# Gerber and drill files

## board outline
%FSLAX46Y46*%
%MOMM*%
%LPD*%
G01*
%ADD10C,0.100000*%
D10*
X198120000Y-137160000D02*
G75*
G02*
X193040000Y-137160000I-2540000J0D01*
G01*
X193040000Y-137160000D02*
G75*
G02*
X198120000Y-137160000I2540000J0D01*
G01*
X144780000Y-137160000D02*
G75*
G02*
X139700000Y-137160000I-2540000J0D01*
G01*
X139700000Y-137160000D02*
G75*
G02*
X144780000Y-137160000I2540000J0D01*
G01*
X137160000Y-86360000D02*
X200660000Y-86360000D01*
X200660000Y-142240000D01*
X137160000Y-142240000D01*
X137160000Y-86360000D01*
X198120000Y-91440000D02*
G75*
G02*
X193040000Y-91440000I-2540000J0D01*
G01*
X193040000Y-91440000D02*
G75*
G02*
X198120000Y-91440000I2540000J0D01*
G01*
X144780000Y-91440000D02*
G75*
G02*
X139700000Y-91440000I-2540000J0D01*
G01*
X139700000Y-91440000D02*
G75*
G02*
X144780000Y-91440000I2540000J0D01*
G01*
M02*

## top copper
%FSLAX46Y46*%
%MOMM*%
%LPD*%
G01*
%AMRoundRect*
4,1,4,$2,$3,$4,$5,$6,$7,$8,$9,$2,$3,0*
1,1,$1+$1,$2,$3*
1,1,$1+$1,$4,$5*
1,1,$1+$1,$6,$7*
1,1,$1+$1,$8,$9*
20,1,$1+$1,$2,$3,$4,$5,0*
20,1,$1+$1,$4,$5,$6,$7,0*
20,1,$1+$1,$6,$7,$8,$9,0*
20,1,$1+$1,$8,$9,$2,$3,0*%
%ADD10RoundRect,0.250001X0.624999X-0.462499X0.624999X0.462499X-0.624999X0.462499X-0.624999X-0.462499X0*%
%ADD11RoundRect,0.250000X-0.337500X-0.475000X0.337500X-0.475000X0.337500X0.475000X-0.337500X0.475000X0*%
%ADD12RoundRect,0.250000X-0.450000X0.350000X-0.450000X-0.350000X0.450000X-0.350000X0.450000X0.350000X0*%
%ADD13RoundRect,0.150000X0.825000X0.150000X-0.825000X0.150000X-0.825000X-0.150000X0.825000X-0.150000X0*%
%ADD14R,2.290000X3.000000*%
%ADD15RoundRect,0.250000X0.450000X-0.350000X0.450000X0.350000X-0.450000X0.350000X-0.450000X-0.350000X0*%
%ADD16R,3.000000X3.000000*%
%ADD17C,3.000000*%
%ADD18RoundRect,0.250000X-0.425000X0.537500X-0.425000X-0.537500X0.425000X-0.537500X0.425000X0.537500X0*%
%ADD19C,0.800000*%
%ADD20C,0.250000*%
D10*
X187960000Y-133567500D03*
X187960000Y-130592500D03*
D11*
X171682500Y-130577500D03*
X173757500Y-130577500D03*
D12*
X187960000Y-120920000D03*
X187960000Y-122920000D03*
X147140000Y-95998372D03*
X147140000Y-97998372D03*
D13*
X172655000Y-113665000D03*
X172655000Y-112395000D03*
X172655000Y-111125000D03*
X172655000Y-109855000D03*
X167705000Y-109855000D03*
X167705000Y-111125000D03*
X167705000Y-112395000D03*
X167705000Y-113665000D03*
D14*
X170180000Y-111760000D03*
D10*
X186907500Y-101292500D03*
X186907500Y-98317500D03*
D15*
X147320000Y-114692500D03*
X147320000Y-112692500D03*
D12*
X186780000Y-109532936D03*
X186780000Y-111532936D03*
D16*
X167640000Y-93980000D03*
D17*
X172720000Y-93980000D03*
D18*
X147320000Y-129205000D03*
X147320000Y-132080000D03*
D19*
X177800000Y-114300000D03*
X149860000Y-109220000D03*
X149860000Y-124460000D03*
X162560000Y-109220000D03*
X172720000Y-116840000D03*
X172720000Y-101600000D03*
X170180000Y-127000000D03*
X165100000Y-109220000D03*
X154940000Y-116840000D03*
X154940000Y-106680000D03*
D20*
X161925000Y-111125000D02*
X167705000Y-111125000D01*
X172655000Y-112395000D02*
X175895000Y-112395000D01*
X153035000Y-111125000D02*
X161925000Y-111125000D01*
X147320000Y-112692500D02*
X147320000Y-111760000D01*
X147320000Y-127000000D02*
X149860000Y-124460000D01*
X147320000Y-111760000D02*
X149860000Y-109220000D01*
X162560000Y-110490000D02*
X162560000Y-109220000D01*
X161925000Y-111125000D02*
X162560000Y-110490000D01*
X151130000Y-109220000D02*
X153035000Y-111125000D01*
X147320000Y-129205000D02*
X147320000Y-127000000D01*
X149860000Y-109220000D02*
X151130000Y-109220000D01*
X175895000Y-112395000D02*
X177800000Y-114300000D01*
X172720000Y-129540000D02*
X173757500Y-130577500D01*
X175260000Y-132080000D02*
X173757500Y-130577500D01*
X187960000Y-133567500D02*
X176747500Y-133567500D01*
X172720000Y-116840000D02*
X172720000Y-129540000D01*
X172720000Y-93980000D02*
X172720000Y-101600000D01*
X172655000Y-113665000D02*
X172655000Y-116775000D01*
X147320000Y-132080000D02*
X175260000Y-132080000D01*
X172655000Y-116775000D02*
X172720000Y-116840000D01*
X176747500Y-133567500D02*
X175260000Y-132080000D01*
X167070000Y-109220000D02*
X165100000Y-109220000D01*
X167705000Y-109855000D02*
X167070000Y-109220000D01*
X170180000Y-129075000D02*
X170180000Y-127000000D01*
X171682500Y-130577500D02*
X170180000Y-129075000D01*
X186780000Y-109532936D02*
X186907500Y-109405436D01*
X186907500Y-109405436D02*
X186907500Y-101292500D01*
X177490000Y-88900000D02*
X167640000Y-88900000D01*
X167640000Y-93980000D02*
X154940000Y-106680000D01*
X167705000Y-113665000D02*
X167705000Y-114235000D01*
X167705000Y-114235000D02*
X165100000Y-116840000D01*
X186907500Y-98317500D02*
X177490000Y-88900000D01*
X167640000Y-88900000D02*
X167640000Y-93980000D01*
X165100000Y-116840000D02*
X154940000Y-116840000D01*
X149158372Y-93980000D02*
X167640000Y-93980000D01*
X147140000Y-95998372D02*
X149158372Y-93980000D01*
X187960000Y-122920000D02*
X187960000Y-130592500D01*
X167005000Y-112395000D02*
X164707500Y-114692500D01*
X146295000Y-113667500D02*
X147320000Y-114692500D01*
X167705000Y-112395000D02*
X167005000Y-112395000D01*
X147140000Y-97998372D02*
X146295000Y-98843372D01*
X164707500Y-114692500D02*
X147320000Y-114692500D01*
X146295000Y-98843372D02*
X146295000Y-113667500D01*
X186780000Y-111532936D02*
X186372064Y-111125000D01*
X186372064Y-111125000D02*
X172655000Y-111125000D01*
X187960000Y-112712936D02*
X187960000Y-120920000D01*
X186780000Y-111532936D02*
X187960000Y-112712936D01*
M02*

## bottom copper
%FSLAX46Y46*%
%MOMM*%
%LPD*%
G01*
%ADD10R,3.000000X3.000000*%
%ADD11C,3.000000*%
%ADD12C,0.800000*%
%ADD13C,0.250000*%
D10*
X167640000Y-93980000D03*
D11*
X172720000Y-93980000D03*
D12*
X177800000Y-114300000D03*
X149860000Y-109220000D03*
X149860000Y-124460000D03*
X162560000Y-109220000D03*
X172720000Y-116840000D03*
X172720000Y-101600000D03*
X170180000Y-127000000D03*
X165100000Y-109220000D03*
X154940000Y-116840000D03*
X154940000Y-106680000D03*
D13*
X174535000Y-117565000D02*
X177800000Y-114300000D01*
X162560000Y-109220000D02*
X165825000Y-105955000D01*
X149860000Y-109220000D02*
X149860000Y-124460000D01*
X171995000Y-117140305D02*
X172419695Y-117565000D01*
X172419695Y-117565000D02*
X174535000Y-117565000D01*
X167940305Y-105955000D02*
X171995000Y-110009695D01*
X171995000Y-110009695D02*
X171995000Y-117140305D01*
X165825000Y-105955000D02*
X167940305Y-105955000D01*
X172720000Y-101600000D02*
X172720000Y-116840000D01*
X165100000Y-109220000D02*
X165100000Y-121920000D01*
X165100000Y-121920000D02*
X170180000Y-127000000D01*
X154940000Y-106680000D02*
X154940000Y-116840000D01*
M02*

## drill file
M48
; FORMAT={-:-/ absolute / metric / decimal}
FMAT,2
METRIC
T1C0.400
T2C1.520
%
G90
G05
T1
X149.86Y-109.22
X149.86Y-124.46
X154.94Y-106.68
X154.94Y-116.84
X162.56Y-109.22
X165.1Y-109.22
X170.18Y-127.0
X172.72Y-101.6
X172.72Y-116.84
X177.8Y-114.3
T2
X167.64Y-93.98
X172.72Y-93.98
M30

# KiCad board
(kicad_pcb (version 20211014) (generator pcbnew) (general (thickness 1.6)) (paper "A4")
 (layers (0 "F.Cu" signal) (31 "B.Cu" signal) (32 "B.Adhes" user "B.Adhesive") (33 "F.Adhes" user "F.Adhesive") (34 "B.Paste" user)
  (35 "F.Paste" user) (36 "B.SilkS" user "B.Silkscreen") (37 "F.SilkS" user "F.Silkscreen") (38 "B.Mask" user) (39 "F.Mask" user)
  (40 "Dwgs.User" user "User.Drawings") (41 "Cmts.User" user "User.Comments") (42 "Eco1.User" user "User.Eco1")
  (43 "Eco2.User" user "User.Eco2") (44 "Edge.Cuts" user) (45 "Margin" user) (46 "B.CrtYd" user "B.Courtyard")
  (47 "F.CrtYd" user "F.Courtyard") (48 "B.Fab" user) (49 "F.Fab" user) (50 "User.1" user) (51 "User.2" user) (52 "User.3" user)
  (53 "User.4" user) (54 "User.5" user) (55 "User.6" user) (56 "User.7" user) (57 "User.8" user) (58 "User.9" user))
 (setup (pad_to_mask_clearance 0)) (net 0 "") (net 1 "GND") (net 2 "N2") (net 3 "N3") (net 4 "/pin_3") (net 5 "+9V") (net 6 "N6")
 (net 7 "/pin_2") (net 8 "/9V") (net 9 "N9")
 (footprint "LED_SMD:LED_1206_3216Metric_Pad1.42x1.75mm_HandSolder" (layer "F.Cu") (at 187.96 132.08 90)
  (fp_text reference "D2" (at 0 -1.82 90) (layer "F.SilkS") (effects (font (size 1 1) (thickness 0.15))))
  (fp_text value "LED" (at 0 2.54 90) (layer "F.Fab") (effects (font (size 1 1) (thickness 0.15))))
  (pad "1" smd roundrect (at -1.4875 0 90) (size 1.425 1.75) (layers "F.Cu" "F.Paste" "F.Mask") (roundrect_rratio 0.175439) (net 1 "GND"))
  (pad "2" smd roundrect (at 1.4875 0 90) (size 1.425 1.75) (layers "F.Cu" "F.Paste" "F.Mask") (roundrect_rratio 0.175439) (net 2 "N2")))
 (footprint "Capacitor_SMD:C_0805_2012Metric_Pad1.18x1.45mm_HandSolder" (layer "F.Cu") (at 172.72 130.5775)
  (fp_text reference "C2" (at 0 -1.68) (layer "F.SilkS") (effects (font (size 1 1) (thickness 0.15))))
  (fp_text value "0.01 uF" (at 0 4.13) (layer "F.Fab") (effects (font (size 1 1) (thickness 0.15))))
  (pad "1" smd roundrect (at -1.0375 0) (size 1.175 1.45) (layers "F.Cu" "F.Paste" "F.Mask") (roundrect_rratio 0.212766) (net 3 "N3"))
  (pad "2" smd roundrect (at 1.0375 0) (size 1.175 1.45) (layers "F.Cu" "F.Paste" "F.Mask") (roundrect_rratio 0.212766) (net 1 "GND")))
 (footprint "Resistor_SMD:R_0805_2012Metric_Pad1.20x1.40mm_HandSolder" (layer "F.Cu") (at 187.96 121.92 -90)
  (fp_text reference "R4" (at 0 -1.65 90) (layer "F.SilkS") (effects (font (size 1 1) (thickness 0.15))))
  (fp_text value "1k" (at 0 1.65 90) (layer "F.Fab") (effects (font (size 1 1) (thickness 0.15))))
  (pad "1" smd roundrect (at -1 0 270) (size 1.2 1.4) (layers "F.Cu" "F.Paste" "F.Mask") (roundrect_rratio 0.208333) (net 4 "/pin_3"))
  (pad "2" smd roundrect (at 1 0 270) (size 1.2 1.4) (layers "F.Cu" "F.Paste" "F.Mask") (roundrect_rratio 0.208333) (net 2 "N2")))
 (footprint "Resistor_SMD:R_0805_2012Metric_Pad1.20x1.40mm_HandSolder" (layer "F.Cu") (at 147.14 96.998372 -90)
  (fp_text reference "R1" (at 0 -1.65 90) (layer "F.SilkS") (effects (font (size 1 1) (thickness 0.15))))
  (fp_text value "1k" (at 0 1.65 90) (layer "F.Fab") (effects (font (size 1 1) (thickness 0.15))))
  (pad "1" smd roundrect (at -1 0 270) (size 1.2 1.4) (layers "F.Cu" "F.Paste" "F.Mask") (roundrect_rratio 0.208333) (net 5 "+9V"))
  (pad "2" smd roundrect (at 1 0 270) (size 1.2 1.4) (layers "F.Cu" "F.Paste" "F.Mask") (roundrect_rratio 0.208333) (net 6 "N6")))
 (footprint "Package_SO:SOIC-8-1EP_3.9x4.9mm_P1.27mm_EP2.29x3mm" (layer "F.Cu") (at 170.18 111.76 180)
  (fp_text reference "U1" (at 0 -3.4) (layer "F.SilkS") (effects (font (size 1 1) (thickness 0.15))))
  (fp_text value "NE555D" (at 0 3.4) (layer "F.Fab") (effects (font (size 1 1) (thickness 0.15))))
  (pad "" smd roundrect (at -0.57 0.75 180) (size 0.92 1.21) (layers "F.Paste") (roundrect_rratio 0.25))
  (pad "" smd roundrect (at 0.57 0.75 180) (size 0.92 1.21) (layers "F.Paste") (roundrect_rratio 0.25))
  (pad "" smd roundrect (at -0.57 -0.75 180) (size 0.92 1.21) (layers "F.Paste") (roundrect_rratio 0.25))
  (pad "" smd roundrect (at 0.57 -0.75 180) (size 0.92 1.21) (layers "F.Paste") (roundrect_rratio 0.25))
  (pad "1" smd roundrect (at -2.475 -1.905 180) (size 1.95 0.6) (layers "F.Cu" "F.Paste" "F.Mask") (roundrect_rratio 0.25) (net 1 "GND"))
  (pad "2" smd roundrect (at -2.475 -0.635 180) (size 1.95 0.6) (layers "F.Cu" "F.Paste" "F.Mask") (roundrect_rratio 0.25) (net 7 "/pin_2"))
  (pad "3" smd roundrect (at -2.475 0.635 180) (size 1.95 0.6) (layers "F.Cu" "F.Paste" "F.Mask") (roundrect_rratio 0.25) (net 4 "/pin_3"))
  (pad "4" smd roundrect (at -2.475 1.905 180) (size 1.95 0.6) (layers "F.Cu" "F.Paste" "F.Mask") (roundrect_rratio 0.25) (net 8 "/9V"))
  (pad "5" smd roundrect (at 2.475 1.905 180) (size 1.95 0.6) (layers "F.Cu" "F.Paste" "F.Mask") (roundrect_rratio 0.25) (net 3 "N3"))
  (pad "6" smd roundrect (at 2.475 0.635 180) (size 1.95 0.6) (layers "F.Cu" "F.Paste" "F.Mask") (roundrect_rratio 0.25) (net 7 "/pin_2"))
  (pad "7" smd roundrect (at 2.475 -0.635 180) (size 1.95 0.6) (layers "F.Cu" "F.Paste" "F.Mask") (roundrect_rratio 0.25) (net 6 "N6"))
  (pad "8" smd roundrect (at 2.475 -1.905 180) (size 1.95 0.6) (layers "F.Cu" "F.Paste" "F.Mask") (roundrect_rratio 0.25) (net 5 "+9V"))
  (pad "9" smd rect (at 0 0 180) (size 2.29 3) (layers "F.Cu" "F.Mask")))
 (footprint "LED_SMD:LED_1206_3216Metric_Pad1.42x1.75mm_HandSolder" (layer "F.Cu") (at 186.9075 99.805 90)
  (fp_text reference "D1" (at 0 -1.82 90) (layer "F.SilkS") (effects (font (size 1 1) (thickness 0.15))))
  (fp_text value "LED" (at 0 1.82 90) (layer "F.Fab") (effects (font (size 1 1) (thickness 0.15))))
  (pad "1" smd roundrect (at -1.4875 0 90) (size 1.425 1.75) (layers "F.Cu" "F.Paste" "F.Mask") (roundrect_rratio 0.175439) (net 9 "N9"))
  (pad "2" smd roundrect (at 1.4875 0 90) (size 1.425 1.75) (layers "F.Cu" "F.Paste" "F.Mask") (roundrect_rratio 0.175439) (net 5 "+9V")))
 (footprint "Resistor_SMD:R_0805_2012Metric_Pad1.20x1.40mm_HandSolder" (layer "F.Cu") (at 147.32 113.6925 90)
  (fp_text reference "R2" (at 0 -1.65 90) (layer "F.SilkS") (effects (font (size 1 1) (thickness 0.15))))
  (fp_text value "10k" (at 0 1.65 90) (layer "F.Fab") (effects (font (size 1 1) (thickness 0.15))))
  (pad "1" smd roundrect (at -1 0 90) (size 1.2 1.4) (layers "F.Cu" "F.Paste" "F.Mask") (roundrect_rratio 0.208333) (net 6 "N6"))
  (pad "2" smd roundrect (at 1 0 90) (size 1.2 1.4) (layers "F.Cu" "F.Paste" "F.Mask") (roundrect_rratio 0.208333) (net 7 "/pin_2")))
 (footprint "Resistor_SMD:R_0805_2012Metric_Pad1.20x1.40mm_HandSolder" (layer "F.Cu") (at 186.78 110.532936 -90)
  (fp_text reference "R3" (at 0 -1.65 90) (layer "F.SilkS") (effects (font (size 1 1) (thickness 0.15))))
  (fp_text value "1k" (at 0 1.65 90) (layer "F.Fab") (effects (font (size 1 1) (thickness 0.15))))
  (pad "1" smd roundrect (at -1 0 270) (size 1.2 1.4) (layers "F.Cu" "F.Paste" "F.Mask") (roundrect_rratio 0.208333) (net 9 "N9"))
  (pad "2" smd roundrect (at 1 0 270) (size 1.2 1.4) (layers "F.Cu" "F.Paste" "F.Mask") (roundrect_rratio 0.208333) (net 4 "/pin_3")))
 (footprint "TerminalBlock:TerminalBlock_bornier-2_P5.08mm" (layer "F.Cu") (at 167.64 93.98)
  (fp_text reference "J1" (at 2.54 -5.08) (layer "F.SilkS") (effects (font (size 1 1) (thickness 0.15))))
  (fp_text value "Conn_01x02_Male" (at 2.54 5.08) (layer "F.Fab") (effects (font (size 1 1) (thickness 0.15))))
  (pad "1" thru_hole rect (at 0 0) (size 3 3) (drill 1.52) (layers *.Cu *.Mask) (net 5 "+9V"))
  (pad "2" thru_hole circle (at 5.08 0) (size 3 3) (drill 1.52) (layers *.Cu *.Mask) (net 1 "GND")))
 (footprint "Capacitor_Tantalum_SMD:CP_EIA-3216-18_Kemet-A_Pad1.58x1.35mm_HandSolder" (layer "F.Cu") (at 147.32 130.6425 -90)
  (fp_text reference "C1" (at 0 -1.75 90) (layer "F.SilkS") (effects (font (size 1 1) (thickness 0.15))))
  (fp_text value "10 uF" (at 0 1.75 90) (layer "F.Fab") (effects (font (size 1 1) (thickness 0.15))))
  (pad "1" smd roundrect (at -1.4375 0 270) (size 1.575 1.35) (layers "F.Cu" "F.Paste" "F.Mask") (roundrect_rratio 0.185185)
   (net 7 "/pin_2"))
  (pad "2" smd roundrect (at 1.4375 0 270) (size 1.575 1.35) (layers "F.Cu" "F.Paste" "F.Mask") (roundrect_rratio 0.185185) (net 1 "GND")))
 (gr_circle (center 195.58 137.16) (end 198.12 137.16) (layer "Edge.Cuts") (width 0.1) (fill none))
 (gr_circle (center 142.24 137.16) (end 139.7 137.16) (layer "Edge.Cuts") (width 0.1) (fill none))
 (gr_rect (start 137.16 86.36) (end 200.66 142.24) (layer "Edge.Cuts") (width 0.1) (fill none))
 (gr_circle (center 195.58 91.44) (end 198.12 91.44) (layer "Edge.Cuts") (width 0.1) (fill none))
 (gr_circle (center 142.24 91.44) (end 144.78 91.44) (layer "Edge.Cuts") (width 0.1) (fill none))
 (segment (start 161.925 111.125) (end 167.705 111.125) (width 0.25) (layer "F.Cu") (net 7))
 (segment (start 172.655 112.395) (end 175.895 112.395) (width 0.25) (layer "F.Cu") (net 7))
 (segment (start 153.035 111.125) (end 161.925 111.125) (width 0.25) (layer "F.Cu") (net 7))
 (segment (start 147.32 112.6925) (end 147.32 111.76) (width 0.25) (layer "F.Cu") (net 7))
 (segment (start 147.32 127) (end 149.86 124.46) (width 0.25) (layer "F.Cu") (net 7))
 (segment (start 147.32 111.76) (end 149.86 109.22) (width 0.25) (layer "F.Cu") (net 7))
 (segment (start 162.56 110.49) (end 162.56 109.22) (width 0.25) (layer "F.Cu") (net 7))
 (segment (start 161.925 111.125) (end 162.56 110.49) (width 0.25) (layer "F.Cu") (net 7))
 (segment (start 151.13 109.22) (end 153.035 111.125) (width 0.25) (layer "F.Cu") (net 7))
 (segment (start 147.32 129.205) (end 147.32 127) (width 0.25) (layer "F.Cu") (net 7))
 (segment (start 149.86 109.22) (end 151.13 109.22) (width 0.25) (layer "F.Cu") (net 7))
 (segment (start 175.895 112.395) (end 177.8 114.3) (width 0.25) (layer "F.Cu") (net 7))
 (via (at 177.8 114.3) (size 0.8) (drill 0.4) (layers "F.Cu" "B.Cu") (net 7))
 (via (at 149.86 109.22) (size 0.8) (drill 0.4) (layers "F.Cu" "B.Cu") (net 7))
 (via (at 149.86 124.46) (size 0.8) (drill 0.4) (layers "F.Cu" "B.Cu") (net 7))
 (via (at 162.56 109.22) (size 0.8) (drill 0.4) (layers "F.Cu" "B.Cu") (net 7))
 (segment (start 174.535 117.565) (end 177.8 114.3) (width 0.25) (layer "B.Cu") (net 7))
 (segment (start 162.56 109.22) (end 165.825 105.955) (width 0.25) (layer "B.Cu") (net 7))
 (segment (start 149.86 109.22) (end 149.86 124.46) (width 0.25) (layer "B.Cu") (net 7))
 (segment (start 171.995 117.140305) (end 172.419695 117.565) (width 0.25) (layer "B.Cu") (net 7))
 (segment (start 172.419695 117.565) (end 174.535 117.565) (width 0.25) (layer "B.Cu") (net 7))
 (segment (start 167.940305 105.955) (end 171.995 110.009695) (width 0.25) (layer "B.Cu") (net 7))
 (segment (start 171.995 110.009695) (end 171.995 117.140305) (width 0.25) (layer "B.Cu") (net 7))
 (segment (start 165.825 105.955) (end 167.940305 105.955) (width 0.25) (layer "B.Cu") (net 7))
 (segment (start 172.72 129.54) (end 173.7575 130.5775) (width 0.25) (layer "F.Cu") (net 1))
 (segment (start 175.26 132.08) (end 173.7575 130.5775) (width 0.25) (layer "F.Cu") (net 1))
 (segment (start 187.96 133.5675) (end 176.7475 133.5675) (width 0.25) (layer "F.Cu") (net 1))
 (segment (start 172.72 116.84) (end 172.72 129.54) (width 0.25) (layer "F.Cu") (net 1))
 (segment (start 172.72 93.98) (end 172.72 101.6) (width 0.25) (layer "F.Cu") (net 1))
 (segment (start 172.655 113.665) (end 172.655 116.775) (width 0.25) (layer "F.Cu") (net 1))
 (segment (start 147.32 132.08) (end 175.26 132.08) (width 0.25) (layer "F.Cu") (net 1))
 (segment (start 172.655 116.775) (end 172.72 116.84) (width 0.25) (layer "F.Cu") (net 1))
 (segment (start 176.7475 133.5675) (end 175.26 132.08) (width 0.25) (layer "F.Cu") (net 1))
 (via (at 172.72 116.84) (size 0.8) (drill 0.4) (layers "F.Cu" "B.Cu") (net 1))
 (via (at 172.72 101.6) (size 0.8) (drill 0.4) (layers "F.Cu" "B.Cu") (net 1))
 (segment (start 172.72 101.6) (end 172.72 116.84) (width 0.25) (layer "B.Cu") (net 1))
 (segment (start 167.07 109.22) (end 165.1 109.22) (width 0.25) (layer "F.Cu") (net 3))
 (segment (start 167.705 109.855) (end 167.07 109.22) (width 0.25) (layer "F.Cu") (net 3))
 (segment (start 170.18 129.075) (end 170.18 127) (width 0.25) (layer "F.Cu") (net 3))
 (segment (start 171.6825 130.5775) (end 170.18 129.075) (width 0.25) (layer "F.Cu") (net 3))
 (via (at 170.18 127) (size 0.8) (drill 0.4) (layers "F.Cu" "B.Cu") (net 3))
 (via (at 165.1 109.22) (size 0.8) (drill 0.4) (layers "F.Cu" "B.Cu") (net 3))
 (segment (start 165.1 109.22) (end 165.1 121.92) (width 0.25) (layer "B.Cu") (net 3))
 (segment (start 165.1 121.92) (end 170.18 127) (width 0.25) (layer "B.Cu") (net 3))
 (segment (start 186.78 109.532936) (end 186.9075 109.405436) (width 0.25) (layer "F.Cu") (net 9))
 (segment (start 186.9075 109.405436) (end 186.9075 101.2925) (width 0.25) (layer "F.Cu") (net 9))
 (segment (start 177.49 88.9) (end 167.64 88.9) (width 0.25) (layer "F.Cu") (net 5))
 (segment (start 167.64 93.98) (end 154.94 106.68) (width 0.25) (layer "F.Cu") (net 5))
 (segment (start 167.705 113.665) (end 167.705 114.235) (width 0.25) (layer "F.Cu") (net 5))
 (segment (start 167.705 114.235) (end 165.1 116.84) (width 0.25) (layer "F.Cu") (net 5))
 (segment (start 186.9075 98.3175) (end 177.49 88.9) (width 0.25) (layer "F.Cu") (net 5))
 (segment (start 167.64 88.9) (end 167.64 93.98) (width 0.25) (layer "F.Cu") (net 5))
 (segment (start 165.1 116.84) (end 154.94 116.84) (width 0.25) (layer "F.Cu") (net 5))
 (segment (start 149.158372 93.98) (end 167.64 93.98) (width 0.25) (layer "F.Cu") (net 5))
 (segment (start 147.14 95.998372) (end 149.158372 93.98) (width 0.25) (layer "F.Cu") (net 5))
 (via (at 154.94 116.84) (size 0.8) (drill 0.4) (layers "F.Cu" "B.Cu") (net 5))
 (via (at 154.94 106.68) (size 0.8) (drill 0.4) (layers "F.Cu" "B.Cu") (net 5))
 (segment (start 154.94 106.68) (end 154.94 116.84) (width 0.25) (layer "B.Cu") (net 5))
 (segment (start 187.96 122.92) (end 187.96 130.5925) (width 0.25) (layer "F.Cu") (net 2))
 (segment (start 167.005 112.395) (end 164.7075 114.6925) (width 0.25) (layer "F.Cu") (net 6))
 (segment (start 146.295 113.6675) (end 147.32 114.6925) (width 0.25) (layer "F.Cu") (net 6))
 (segment (start 167.705 112.395) (end 167.005 112.395) (width 0.25) (layer "F.Cu") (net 6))
 (segment (start 147.14 97.998372) (end 146.295 98.843372) (width 0.25) (layer "F.Cu") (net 6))
 (segment (start 164.7075 114.6925) (end 147.32 114.6925) (width 0.25) (layer "F.Cu") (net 6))
 (segment (start 146.295 98.843372) (end 146.295 113.6675) (width 0.25) (layer "F.Cu") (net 6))
 (segment (start 186.78 111.532936) (end 186.372064 111.125) (width 0.25) (layer "F.Cu") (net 4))
 (segment (start 186.372064 111.125) (end 172.655 111.125) (width 0.25) (layer "F.Cu") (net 4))
 (segment (start 187.96 112.712936) (end 187.96 120.92) (width 0.25) (layer "F.Cu") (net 4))
 (segment (start 186.78 111.532936) (end 187.96 112.712936) (width 0.25) (layer "F.Cu") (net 4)))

